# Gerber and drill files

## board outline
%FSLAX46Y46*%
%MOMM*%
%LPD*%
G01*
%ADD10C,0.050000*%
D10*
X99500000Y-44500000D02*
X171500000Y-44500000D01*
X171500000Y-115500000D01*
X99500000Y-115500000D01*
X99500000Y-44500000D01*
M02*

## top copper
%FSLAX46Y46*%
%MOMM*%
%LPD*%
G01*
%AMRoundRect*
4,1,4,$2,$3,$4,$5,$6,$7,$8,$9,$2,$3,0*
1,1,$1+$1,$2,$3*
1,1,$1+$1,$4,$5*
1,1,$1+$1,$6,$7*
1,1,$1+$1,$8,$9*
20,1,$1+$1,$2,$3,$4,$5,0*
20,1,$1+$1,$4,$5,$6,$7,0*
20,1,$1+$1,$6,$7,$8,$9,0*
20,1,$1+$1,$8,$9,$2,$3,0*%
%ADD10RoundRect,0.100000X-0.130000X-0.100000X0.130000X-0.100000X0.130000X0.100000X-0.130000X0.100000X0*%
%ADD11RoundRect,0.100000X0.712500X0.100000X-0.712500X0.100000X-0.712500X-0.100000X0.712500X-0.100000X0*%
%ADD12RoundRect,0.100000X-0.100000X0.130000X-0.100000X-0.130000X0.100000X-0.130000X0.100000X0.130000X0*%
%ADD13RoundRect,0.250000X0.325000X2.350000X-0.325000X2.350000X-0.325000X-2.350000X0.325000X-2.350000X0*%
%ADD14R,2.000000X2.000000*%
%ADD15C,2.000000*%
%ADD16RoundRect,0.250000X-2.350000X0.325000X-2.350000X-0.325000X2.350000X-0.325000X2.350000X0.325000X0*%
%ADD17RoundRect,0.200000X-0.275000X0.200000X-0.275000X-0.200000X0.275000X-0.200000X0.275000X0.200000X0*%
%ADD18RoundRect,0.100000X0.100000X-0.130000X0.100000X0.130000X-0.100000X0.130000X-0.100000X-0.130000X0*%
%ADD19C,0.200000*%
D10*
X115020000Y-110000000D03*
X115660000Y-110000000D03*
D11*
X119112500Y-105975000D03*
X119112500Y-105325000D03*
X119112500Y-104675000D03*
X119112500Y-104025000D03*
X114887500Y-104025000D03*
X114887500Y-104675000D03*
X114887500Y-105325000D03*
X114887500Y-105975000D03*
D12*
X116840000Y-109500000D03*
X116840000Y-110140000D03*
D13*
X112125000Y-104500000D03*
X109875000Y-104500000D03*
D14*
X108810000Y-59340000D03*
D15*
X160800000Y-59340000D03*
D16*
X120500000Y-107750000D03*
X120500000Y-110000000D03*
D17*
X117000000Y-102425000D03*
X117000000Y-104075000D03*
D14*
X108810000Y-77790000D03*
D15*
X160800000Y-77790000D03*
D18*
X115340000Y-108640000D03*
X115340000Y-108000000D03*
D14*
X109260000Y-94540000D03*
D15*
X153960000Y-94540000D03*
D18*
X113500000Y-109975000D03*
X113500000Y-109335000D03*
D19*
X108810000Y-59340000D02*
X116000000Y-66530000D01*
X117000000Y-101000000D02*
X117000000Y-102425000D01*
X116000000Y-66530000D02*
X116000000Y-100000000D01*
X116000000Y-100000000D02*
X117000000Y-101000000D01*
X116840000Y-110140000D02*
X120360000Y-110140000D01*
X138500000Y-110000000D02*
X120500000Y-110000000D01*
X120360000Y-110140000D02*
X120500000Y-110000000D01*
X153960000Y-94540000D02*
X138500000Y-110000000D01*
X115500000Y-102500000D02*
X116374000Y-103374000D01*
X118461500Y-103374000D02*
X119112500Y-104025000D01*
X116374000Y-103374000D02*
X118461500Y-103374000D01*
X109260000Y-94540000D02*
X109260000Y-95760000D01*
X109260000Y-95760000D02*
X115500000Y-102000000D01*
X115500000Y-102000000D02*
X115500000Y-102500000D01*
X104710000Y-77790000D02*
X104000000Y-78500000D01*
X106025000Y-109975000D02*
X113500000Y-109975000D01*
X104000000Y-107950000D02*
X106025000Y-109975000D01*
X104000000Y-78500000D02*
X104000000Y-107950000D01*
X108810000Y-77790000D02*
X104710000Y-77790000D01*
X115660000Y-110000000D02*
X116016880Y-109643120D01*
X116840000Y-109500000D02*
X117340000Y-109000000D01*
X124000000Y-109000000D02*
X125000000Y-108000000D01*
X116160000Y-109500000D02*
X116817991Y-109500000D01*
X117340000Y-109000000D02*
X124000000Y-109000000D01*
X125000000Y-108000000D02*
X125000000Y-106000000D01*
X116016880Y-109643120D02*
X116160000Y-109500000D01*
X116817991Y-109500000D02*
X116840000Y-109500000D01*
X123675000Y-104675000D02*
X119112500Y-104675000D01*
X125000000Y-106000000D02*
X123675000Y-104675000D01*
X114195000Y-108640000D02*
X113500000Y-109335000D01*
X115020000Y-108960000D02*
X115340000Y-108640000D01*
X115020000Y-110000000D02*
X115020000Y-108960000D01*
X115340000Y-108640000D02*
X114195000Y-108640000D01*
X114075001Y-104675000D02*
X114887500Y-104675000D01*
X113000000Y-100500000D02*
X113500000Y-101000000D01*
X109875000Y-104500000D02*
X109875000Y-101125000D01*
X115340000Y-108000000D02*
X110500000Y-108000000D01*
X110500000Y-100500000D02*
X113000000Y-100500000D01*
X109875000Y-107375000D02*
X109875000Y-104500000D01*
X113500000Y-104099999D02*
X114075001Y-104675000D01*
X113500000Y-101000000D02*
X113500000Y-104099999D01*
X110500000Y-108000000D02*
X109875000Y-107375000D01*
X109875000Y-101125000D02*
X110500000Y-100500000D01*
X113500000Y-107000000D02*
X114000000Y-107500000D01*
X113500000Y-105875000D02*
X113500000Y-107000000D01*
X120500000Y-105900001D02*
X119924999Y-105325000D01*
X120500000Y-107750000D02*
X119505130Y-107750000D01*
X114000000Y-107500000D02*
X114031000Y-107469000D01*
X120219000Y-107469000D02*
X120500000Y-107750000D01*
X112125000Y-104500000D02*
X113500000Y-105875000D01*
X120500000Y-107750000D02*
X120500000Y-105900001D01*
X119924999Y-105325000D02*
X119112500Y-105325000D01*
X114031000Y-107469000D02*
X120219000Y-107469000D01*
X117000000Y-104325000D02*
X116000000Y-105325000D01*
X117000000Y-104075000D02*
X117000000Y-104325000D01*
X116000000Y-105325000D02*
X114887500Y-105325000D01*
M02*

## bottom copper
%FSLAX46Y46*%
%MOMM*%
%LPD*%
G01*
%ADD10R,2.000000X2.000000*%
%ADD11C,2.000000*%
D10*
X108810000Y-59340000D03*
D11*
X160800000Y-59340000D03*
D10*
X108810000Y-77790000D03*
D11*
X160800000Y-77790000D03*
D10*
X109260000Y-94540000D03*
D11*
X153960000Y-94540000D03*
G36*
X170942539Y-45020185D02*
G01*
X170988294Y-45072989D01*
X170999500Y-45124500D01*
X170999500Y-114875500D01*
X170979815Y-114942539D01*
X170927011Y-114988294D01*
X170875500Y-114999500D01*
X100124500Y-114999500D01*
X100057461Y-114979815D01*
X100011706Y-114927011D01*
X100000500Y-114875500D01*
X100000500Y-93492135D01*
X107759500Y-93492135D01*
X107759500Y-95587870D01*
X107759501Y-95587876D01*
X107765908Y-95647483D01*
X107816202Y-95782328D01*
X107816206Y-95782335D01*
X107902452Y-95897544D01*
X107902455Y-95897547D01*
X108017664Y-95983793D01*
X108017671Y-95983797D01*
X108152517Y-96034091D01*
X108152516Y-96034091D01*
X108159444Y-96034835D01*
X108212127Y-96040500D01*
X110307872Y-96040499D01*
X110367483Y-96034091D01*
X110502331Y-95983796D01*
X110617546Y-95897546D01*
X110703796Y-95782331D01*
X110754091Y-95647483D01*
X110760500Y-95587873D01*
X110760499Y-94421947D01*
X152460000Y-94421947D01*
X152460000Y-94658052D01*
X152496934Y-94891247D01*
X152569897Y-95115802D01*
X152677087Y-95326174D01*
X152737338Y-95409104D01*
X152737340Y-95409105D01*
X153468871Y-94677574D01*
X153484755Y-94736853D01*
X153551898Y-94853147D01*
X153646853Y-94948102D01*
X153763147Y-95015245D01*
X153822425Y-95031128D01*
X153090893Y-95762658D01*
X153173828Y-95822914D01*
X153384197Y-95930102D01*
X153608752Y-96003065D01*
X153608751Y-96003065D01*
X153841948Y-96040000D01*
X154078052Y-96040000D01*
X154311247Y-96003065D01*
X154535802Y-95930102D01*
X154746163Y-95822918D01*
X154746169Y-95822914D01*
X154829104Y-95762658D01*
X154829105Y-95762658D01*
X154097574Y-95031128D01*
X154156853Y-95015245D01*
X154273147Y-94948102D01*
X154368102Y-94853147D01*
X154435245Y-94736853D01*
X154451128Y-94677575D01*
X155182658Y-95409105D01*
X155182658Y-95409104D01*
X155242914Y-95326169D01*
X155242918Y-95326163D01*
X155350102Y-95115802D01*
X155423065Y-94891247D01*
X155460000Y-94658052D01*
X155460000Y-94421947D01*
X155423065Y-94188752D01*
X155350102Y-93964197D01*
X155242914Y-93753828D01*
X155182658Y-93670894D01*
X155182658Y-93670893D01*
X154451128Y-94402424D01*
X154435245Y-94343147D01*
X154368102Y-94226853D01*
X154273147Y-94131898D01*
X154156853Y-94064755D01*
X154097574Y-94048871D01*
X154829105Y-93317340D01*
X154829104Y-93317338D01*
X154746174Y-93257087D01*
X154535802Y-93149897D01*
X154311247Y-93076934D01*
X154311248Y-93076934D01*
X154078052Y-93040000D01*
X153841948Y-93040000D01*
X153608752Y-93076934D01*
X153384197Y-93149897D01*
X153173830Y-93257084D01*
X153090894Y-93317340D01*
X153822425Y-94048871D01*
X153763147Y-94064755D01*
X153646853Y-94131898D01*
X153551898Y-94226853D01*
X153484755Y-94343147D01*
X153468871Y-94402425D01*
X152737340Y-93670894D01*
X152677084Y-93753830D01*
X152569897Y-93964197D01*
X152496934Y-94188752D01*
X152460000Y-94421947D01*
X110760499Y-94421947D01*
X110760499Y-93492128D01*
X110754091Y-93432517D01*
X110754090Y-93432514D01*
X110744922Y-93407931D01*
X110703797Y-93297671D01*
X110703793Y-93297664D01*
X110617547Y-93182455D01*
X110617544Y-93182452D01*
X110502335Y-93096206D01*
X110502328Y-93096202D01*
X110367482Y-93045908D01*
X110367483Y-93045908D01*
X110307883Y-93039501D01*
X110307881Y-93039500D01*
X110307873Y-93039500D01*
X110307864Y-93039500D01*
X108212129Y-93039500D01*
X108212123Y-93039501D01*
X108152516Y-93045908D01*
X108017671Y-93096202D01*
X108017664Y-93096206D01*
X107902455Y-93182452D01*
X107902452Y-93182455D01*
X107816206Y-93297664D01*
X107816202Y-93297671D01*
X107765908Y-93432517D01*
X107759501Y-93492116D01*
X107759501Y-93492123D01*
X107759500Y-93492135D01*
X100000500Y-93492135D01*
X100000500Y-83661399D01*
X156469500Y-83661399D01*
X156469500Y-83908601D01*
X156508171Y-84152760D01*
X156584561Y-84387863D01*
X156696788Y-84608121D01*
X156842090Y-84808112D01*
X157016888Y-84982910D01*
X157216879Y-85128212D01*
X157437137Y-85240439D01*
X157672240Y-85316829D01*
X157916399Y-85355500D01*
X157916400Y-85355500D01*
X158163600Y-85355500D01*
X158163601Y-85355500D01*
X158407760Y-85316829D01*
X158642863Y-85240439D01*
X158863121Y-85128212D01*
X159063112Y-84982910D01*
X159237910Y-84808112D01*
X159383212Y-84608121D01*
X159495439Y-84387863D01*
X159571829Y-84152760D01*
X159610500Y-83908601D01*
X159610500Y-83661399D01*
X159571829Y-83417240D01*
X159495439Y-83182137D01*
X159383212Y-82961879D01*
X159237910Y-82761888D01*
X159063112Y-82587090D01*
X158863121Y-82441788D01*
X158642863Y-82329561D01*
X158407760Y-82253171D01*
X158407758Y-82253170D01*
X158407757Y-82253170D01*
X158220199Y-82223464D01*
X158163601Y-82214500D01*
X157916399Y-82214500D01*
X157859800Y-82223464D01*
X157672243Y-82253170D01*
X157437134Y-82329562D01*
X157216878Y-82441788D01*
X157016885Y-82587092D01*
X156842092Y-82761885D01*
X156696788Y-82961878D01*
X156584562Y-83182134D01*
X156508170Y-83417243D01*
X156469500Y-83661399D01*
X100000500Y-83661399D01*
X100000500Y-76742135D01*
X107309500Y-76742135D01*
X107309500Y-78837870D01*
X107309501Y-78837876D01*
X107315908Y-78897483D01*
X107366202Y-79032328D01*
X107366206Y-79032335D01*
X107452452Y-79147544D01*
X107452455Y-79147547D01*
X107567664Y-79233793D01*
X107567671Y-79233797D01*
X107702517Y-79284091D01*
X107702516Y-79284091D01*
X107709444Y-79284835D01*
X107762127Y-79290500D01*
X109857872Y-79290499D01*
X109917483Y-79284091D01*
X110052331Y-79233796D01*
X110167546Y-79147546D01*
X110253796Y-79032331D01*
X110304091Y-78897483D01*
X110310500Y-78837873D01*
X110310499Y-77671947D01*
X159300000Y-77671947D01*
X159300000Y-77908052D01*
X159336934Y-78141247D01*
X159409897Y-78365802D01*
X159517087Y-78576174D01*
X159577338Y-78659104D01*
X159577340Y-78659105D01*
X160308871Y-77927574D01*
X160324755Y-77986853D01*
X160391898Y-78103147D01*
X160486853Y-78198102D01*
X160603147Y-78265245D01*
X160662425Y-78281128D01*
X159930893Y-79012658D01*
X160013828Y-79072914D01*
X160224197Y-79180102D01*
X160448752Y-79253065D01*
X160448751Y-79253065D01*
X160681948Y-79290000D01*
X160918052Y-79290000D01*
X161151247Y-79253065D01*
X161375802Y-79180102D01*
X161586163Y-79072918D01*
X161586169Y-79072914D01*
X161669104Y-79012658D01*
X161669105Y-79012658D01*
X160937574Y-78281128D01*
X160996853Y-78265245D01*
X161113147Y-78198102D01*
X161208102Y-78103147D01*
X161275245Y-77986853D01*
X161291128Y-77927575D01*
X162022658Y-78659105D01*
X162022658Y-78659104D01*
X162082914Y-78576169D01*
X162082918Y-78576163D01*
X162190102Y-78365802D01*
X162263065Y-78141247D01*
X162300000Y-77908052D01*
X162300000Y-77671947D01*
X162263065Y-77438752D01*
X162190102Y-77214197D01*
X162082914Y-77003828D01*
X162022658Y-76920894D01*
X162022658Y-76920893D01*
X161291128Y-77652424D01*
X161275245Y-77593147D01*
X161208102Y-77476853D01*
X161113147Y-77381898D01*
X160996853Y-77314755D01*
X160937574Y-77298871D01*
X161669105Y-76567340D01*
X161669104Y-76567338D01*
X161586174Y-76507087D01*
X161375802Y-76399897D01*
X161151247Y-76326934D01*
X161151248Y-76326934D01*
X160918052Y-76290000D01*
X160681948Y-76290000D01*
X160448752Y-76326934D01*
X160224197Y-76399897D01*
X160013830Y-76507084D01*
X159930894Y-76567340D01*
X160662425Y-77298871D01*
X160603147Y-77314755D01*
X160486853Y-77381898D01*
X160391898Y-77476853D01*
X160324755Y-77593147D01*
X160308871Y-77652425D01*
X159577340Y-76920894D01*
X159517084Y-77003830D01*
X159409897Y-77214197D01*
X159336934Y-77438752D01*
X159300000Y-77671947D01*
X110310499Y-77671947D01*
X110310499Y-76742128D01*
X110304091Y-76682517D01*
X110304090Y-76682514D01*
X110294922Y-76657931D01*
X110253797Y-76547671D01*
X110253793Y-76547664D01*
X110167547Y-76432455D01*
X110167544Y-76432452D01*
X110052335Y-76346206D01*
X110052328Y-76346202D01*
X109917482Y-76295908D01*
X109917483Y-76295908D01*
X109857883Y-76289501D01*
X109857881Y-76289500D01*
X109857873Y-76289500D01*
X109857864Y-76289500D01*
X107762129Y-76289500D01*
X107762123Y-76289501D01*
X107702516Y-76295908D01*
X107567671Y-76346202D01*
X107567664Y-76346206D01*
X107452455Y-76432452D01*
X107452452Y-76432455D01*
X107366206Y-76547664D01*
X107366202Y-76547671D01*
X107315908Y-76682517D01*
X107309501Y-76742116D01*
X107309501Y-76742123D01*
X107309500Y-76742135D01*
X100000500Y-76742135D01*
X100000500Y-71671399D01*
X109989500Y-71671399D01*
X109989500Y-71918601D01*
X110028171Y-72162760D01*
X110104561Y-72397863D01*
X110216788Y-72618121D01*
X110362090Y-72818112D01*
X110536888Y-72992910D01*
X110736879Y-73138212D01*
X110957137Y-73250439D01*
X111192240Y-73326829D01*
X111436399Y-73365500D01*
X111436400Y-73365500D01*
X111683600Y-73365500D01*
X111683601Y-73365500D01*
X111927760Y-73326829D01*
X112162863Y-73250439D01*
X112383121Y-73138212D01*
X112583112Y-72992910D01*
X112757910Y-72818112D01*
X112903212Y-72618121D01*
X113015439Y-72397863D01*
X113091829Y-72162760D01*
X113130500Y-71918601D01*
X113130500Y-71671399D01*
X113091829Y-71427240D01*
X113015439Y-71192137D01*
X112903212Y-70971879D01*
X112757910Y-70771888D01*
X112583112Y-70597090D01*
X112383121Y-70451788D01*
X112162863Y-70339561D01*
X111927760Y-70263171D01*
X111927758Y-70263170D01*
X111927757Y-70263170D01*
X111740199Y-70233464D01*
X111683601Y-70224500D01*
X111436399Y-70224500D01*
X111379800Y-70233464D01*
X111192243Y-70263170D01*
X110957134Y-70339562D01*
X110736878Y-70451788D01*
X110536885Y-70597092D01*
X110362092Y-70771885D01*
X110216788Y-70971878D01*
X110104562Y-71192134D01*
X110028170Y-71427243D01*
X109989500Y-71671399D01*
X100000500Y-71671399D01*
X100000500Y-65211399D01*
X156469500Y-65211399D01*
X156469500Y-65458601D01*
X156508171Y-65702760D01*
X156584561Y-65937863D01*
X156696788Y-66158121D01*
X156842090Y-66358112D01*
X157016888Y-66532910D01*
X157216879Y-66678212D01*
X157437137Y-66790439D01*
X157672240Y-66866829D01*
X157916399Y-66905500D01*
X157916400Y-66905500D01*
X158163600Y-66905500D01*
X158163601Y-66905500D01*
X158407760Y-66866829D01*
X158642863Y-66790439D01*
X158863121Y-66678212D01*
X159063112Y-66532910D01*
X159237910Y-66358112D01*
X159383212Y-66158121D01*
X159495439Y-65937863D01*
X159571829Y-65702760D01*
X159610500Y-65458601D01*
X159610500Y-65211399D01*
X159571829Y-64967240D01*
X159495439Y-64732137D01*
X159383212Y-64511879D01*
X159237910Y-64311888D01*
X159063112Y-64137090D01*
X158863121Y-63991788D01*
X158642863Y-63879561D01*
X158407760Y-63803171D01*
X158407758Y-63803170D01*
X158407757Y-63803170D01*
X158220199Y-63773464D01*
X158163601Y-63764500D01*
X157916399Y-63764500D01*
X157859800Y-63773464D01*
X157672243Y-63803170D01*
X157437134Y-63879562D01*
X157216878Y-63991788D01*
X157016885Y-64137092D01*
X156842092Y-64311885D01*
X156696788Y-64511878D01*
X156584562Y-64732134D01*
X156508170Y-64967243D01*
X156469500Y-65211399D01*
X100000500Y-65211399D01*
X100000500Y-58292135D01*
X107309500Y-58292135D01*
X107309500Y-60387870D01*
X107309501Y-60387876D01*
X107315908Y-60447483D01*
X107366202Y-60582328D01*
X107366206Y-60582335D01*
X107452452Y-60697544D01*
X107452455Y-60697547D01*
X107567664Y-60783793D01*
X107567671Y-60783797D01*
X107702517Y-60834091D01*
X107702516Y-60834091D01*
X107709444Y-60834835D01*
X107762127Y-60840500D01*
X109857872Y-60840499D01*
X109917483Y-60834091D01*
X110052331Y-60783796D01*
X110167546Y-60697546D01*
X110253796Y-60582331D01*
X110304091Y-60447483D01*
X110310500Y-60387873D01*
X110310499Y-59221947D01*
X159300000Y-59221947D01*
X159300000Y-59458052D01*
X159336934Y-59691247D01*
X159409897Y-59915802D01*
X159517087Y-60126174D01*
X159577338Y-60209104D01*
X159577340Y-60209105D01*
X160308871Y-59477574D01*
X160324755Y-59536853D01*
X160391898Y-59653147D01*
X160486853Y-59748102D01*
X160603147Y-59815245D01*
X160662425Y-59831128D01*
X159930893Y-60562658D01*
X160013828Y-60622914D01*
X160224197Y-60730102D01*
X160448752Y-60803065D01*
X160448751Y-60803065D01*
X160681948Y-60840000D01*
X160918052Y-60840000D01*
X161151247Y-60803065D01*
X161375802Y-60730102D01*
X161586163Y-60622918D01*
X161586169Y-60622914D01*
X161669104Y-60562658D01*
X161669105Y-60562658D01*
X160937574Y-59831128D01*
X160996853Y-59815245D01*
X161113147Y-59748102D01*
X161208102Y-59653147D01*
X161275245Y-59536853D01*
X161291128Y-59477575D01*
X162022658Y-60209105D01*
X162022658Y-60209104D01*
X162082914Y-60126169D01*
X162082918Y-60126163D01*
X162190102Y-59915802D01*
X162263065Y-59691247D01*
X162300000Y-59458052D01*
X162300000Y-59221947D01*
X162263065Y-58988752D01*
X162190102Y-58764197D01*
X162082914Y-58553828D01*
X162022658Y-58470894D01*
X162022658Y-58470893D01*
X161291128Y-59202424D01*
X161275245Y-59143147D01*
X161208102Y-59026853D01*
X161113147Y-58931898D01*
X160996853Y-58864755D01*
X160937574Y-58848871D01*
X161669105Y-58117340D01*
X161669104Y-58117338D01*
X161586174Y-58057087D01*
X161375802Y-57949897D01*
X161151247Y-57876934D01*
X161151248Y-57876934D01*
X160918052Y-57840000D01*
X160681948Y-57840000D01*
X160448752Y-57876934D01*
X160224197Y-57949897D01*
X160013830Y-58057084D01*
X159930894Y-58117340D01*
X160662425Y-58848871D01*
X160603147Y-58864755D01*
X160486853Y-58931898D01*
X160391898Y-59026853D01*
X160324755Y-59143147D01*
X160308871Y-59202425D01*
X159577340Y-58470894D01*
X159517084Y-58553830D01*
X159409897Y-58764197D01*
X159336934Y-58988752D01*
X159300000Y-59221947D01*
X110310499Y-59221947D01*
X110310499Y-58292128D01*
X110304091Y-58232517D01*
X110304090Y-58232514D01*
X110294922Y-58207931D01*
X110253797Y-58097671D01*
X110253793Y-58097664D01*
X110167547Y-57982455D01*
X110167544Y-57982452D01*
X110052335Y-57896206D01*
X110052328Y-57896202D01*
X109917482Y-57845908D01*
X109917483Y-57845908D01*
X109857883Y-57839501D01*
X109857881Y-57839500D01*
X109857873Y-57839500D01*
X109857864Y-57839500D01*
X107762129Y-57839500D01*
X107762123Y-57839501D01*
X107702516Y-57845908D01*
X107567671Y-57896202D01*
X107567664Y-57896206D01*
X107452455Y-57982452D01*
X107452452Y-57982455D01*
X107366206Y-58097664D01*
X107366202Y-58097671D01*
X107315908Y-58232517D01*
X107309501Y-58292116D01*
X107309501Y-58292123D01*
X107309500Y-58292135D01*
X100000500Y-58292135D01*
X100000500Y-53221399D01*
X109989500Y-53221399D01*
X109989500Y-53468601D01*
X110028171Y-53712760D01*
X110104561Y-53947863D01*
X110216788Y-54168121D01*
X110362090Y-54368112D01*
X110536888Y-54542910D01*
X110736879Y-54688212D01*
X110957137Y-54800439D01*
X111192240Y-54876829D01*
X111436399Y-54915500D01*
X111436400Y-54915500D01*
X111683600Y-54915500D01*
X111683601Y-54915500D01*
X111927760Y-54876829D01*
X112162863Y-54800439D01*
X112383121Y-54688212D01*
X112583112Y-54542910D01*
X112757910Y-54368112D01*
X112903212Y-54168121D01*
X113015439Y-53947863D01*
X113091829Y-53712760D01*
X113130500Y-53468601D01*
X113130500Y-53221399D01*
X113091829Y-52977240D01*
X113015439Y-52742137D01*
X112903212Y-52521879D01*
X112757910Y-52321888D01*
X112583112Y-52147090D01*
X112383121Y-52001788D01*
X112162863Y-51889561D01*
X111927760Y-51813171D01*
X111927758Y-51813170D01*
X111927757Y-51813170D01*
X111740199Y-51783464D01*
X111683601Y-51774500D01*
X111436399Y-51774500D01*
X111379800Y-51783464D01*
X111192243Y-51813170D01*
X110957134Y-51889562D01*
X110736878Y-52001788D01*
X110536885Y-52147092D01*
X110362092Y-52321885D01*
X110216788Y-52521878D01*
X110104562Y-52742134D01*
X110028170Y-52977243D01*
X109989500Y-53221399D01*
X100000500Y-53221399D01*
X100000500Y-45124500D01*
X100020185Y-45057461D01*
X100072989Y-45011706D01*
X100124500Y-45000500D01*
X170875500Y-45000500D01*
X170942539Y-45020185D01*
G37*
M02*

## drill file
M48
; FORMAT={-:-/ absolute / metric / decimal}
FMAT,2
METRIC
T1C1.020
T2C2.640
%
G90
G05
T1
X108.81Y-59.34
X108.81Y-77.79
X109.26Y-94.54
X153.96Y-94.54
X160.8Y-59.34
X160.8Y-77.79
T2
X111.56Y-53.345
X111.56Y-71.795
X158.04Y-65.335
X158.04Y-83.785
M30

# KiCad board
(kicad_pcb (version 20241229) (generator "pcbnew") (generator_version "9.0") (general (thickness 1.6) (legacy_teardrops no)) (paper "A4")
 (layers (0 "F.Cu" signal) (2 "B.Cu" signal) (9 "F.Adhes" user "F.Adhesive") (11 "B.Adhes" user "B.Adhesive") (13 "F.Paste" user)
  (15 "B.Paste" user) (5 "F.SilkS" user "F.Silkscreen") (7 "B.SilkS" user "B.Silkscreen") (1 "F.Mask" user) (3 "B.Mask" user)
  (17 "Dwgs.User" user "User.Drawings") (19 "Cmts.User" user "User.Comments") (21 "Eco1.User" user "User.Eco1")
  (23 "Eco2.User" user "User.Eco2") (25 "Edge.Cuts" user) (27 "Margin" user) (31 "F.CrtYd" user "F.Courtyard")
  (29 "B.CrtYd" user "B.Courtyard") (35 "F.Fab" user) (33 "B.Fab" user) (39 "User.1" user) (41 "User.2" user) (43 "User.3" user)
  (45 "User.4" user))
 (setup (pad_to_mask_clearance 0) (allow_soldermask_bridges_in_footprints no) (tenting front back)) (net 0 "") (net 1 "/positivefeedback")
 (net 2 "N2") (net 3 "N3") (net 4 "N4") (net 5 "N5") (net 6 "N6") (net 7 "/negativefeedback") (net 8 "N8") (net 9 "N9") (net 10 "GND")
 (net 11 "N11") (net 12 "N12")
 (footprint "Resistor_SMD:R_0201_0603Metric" (layer "F.Cu") (at 115.34 110)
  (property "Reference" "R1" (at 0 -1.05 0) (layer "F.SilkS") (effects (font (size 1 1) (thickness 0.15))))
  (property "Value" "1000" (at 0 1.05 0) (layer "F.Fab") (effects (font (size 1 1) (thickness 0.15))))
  (pad "" smd roundrect (at -0.345 0) (size 0.318 0.36) (layers "F.Paste") (roundrect_rratio 0.25))
  (pad "" smd roundrect (at 0.345 0) (size 0.318 0.36) (layers "F.Paste") (roundrect_rratio 0.25))
  (pad "1" smd roundrect (at -0.32 0) (size 0.46 0.4) (layers "F.Cu" "F.Mask") (roundrect_rratio 0.25) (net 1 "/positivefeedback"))
  (pad "2" smd roundrect (at 0.32 0) (size 0.46 0.4) (layers "F.Cu" "F.Mask") (roundrect_rratio 0.25) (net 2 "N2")))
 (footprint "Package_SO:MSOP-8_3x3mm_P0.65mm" (layer "F.Cu") (at 117 105 180)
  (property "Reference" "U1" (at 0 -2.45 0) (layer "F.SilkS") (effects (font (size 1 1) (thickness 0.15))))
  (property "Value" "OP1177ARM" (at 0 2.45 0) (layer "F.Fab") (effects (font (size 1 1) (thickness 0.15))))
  (pad "1" smd roundrect (at -2.1125 -0.975 180) (size 1.625 0.4) (layers "F.Cu" "F.Mask" "F.Paste") (roundrect_rratio 0.25) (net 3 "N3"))
  (pad "2" smd roundrect (at -2.1125 -0.325 180) (size 1.625 0.4) (layers "F.Cu" "F.Mask" "F.Paste") (roundrect_rratio 0.25) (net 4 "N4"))
  (pad "3" smd roundrect (at -2.1125 0.325 180) (size 1.625 0.4) (layers "F.Cu" "F.Mask" "F.Paste") (roundrect_rratio 0.25) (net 2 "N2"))
  (pad "4" smd roundrect (at -2.1125 0.975 180) (size 1.625 0.4) (layers "F.Cu" "F.Mask" "F.Paste") (roundrect_rratio 0.25) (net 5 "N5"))
  (pad "5" smd roundrect (at 2.1125 0.975 180) (size 1.625 0.4) (layers "F.Cu" "F.Mask" "F.Paste") (roundrect_rratio 0.25) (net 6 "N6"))
  (pad "6" smd roundrect (at 2.1125 0.325 180) (size 1.625 0.4) (layers "F.Cu" "F.Mask" "F.Paste") (roundrect_rratio 0.25)
   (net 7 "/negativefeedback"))
  (pad "7" smd roundrect (at 2.1125 -0.325 180) (size 1.625 0.4) (layers "F.Cu" "F.Mask" "F.Paste") (roundrect_rratio 0.25) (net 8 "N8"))
  (pad "8" smd roundrect (at 2.1125 -0.975 180) (size 1.625 0.4) (layers "F.Cu" "F.Mask" "F.Paste") (roundrect_rratio 0.25) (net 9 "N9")))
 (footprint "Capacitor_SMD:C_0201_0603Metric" (layer "F.Cu") (at 116.84 109.82 -90)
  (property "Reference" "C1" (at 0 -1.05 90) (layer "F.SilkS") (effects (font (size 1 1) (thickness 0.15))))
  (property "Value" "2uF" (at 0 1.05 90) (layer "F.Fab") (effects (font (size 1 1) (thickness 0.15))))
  (pad "" smd roundrect (at -0.345 0 270) (size 0.318 0.36) (layers "F.Paste") (roundrect_rratio 0.25))
  (pad "" smd roundrect (at 0.345 0 270) (size 0.318 0.36) (layers "F.Paste") (roundrect_rratio 0.25))
  (pad "1" smd roundrect (at -0.32 0 270) (size 0.46 0.4) (layers "F.Cu" "F.Mask") (roundrect_rratio 0.25) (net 2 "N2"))
  (pad "2" smd roundrect (at 0.32 0 270) (size 0.46 0.4) (layers "F.Cu" "F.Mask") (roundrect_rratio 0.25) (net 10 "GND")))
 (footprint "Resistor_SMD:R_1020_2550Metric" (layer "F.Cu") (at 111 104.5 180)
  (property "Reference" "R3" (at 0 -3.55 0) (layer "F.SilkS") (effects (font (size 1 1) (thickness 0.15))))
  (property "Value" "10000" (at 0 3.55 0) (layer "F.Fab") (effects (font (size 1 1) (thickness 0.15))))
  (pad "1" smd roundrect (at -1.125 0 180) (size 1.15 5.2) (layers "F.Cu" "F.Mask" "F.Paste") (roundrect_rratio 0.217391) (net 4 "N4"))
  (pad "2" smd roundrect (at 1.125 0 180) (size 1.15 5.2) (layers "F.Cu" "F.Mask" "F.Paste") (roundrect_rratio 0.217391)
   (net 7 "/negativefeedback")))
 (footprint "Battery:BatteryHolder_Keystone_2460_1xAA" (layer "F.Cu") (at 108.81 59.34)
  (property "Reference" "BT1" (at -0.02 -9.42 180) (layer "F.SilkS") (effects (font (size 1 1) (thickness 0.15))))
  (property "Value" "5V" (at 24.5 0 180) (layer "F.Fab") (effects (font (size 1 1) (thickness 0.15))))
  (pad "" np_thru_hole circle (at 2.75 -5.995 90) (size 2.64 2.64) (drill 2.64) (layers "*.Cu" "*.Mask"))
  (pad "" np_thru_hole circle (at 49.23 5.995) (size 2.64 2.64) (drill 2.64) (layers "*.Cu" "*.Mask"))
  (pad "1" thru_hole rect (at 0 0 180) (size 2 2) (drill 1.02) (layers "*.Cu" "*.Mask") (remove_unused_layers no) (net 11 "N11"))
  (pad "2" thru_hole circle (at 51.99 0 180) (size 2 2) (drill 1.02) (layers "*.Cu" "*.Mask") (remove_unused_layers no) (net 10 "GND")))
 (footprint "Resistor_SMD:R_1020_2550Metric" (layer "F.Cu") (at 120.5 108.875 -90)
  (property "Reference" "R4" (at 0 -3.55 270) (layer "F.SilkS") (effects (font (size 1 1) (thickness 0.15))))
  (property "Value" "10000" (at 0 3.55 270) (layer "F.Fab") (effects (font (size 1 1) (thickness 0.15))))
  (pad "1" smd roundrect (at -1.125 0 270) (size 1.15 5.2) (layers "F.Cu" "F.Mask" "F.Paste") (roundrect_rratio 0.217391) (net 4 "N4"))
  (pad "2" smd roundrect (at 1.125 0 270) (size 1.15 5.2) (layers "F.Cu" "F.Mask" "F.Paste") (roundrect_rratio 0.217391) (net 10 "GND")))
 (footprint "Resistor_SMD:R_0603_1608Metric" (layer "F.Cu") (at 117 103.25 -90)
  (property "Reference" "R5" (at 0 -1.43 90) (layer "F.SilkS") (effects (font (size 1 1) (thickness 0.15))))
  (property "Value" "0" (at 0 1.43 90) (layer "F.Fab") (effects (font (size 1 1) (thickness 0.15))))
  (pad "1" smd roundrect (at -0.825 0 270) (size 0.8 0.95) (layers "F.Cu" "F.Mask" "F.Paste") (roundrect_rratio 0.25) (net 11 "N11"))
  (pad "2" smd roundrect (at 0.825 0 270) (size 0.8 0.95) (layers "F.Cu" "F.Mask" "F.Paste") (roundrect_rratio 0.25) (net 8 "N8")))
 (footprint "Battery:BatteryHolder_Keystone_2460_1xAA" (layer "F.Cu") (at 108.81 77.79)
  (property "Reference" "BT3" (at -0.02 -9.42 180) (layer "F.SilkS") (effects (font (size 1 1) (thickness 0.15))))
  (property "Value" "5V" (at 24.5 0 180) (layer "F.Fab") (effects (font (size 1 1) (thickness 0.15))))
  (pad "" np_thru_hole circle (at 2.75 -5.995 90) (size 2.64 2.64) (drill 2.64) (layers "*.Cu" "*.Mask"))
  (pad "" np_thru_hole circle (at 49.23 5.995) (size 2.64 2.64) (drill 2.64) (layers "*.Cu" "*.Mask"))
  (pad "1" thru_hole rect (at 0 0 180) (size 2 2) (drill 1.02) (layers "*.Cu" "*.Mask") (remove_unused_layers no) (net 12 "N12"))
  (pad "2" thru_hole circle (at 51.99 0 180) (size 2 2) (drill 1.02) (layers "*.Cu" "*.Mask") (remove_unused_layers no) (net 10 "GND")))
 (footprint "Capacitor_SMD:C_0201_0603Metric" (layer "F.Cu") (at 115.34 108.32 90)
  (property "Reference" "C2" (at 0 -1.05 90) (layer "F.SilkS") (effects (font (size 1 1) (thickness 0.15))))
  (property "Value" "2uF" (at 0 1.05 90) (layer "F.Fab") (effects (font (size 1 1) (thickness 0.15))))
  (pad "" smd roundrect (at -0.345 0 90) (size 0.318 0.36) (layers "F.Paste") (roundrect_rratio 0.25))
  (pad "" smd roundrect (at 0.345 0 90) (size 0.318 0.36) (layers "F.Paste") (roundrect_rratio 0.25))
  (pad "1" smd roundrect (at -0.32 0 90) (size 0.46 0.4) (layers "F.Cu" "F.Mask") (roundrect_rratio 0.25) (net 1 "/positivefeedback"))
  (pad "2" smd roundrect (at 0.32 0 90) (size 0.46 0.4) (layers "F.Cu" "F.Mask") (roundrect_rratio 0.25) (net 7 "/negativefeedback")))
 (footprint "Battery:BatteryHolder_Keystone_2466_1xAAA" (layer "F.Cu") (at 109.26 94.54)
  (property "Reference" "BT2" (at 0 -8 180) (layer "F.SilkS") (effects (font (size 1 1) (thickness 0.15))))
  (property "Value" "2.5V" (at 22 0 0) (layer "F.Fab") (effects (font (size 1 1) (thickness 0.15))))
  (pad "1" thru_hole rect (at 0 0) (size 2 2) (drill 1.02) (layers "*.Cu" "*.Mask") (remove_unused_layers no) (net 5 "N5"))
  (pad "2" thru_hole circle (at 44.7 0) (size 2 2) (drill 1.02) (layers "*.Cu" "*.Mask") (remove_unused_layers no) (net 10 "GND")))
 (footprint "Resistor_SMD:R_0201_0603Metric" (layer "F.Cu") (at 113.5 109.655 90)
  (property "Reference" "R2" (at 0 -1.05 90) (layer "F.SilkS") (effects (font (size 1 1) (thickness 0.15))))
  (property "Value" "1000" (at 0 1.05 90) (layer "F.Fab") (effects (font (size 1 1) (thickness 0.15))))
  (pad "" smd roundrect (at -0.345 0 90) (size 0.318 0.36) (layers "F.Paste") (roundrect_rratio 0.25))
  (pad "" smd roundrect (at 0.345 0 90) (size 0.318 0.36) (layers "F.Paste") (roundrect_rratio 0.25))
  (pad "1" smd roundrect (at -0.32 0 90) (size 0.46 0.4) (layers "F.Cu" "F.Mask") (roundrect_rratio 0.25) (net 12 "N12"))
  (pad "2" smd roundrect (at 0.32 0 90) (size 0.46 0.4) (layers "F.Cu" "F.Mask") (roundrect_rratio 0.25) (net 1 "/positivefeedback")))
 (gr_rect (start 99.5 44.5) (end 171.5 115.5) (stroke (width 0.05) (type default)) (fill no) (layer "Edge.Cuts"))
 (segment (start 108.81 59.34) (end 116 66.53) (width 0.2) (layer "F.Cu") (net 11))
 (segment (start 117 101) (end 117 102.425) (width 0.2) (layer "F.Cu") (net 11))
 (segment (start 116 66.53) (end 116 100) (width 0.2) (layer "F.Cu") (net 11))
 (segment (start 116 100) (end 117 101) (width 0.2) (layer "F.Cu") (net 11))
 (segment (start 116.84 110.14) (end 120.36 110.14) (width 0.2) (layer "F.Cu") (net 10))
 (segment (start 138.5 110) (end 120.5 110) (width 0.2) (layer "F.Cu") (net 10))
 (segment (start 120.36 110.14) (end 120.5 110) (width 0.2) (layer "F.Cu") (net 10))
 (segment (start 153.96 94.54) (end 138.5 110) (width 0.2) (layer "F.Cu") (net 10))
 (segment (start 115.5 102.5) (end 116.374 103.374) (width 0.2) (layer "F.Cu") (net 5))
 (segment (start 118.4615 103.374) (end 119.1125 104.025) (width 0.2) (layer "F.Cu") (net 5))
 (segment (start 116.374 103.374) (end 118.4615 103.374) (width 0.2) (layer "F.Cu") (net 5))
 (segment (start 109.26 94.54) (end 109.26 95.76) (width 0.2) (layer "F.Cu") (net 5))
 (segment (start 109.26 95.76) (end 115.5 102) (width 0.2) (layer "F.Cu") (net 5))
 (segment (start 115.5 102) (end 115.5 102.5) (width 0.2) (layer "F.Cu") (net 5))
 (segment (start 104.71 77.79) (end 104 78.5) (width 0.2) (layer "F.Cu") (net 12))
 (segment (start 106.025 109.975) (end 113.5 109.975) (width 0.2) (layer "F.Cu") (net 12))
 (segment (start 104 107.95) (end 106.025 109.975) (width 0.2) (layer "F.Cu") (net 12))
 (segment (start 104 78.5) (end 104 107.95) (width 0.2) (layer "F.Cu") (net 12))
 (segment (start 108.81 77.79) (end 104.71 77.79) (width 0.2) (layer "F.Cu") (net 12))
 (segment (start 115.66 110) (end 116.01688 109.64312) (width 0.2) (layer "F.Cu") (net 2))
 (segment (start 116.84 109.5) (end 117.34 109) (width 0.2) (layer "F.Cu") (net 2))
 (segment (start 124 109) (end 125 108) (width 0.2) (layer "F.Cu") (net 2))
 (segment (start 116.16 109.5) (end 116.817991 109.5) (width 0.2) (layer "F.Cu") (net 2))
 (segment (start 117.34 109) (end 124 109) (width 0.2) (layer "F.Cu") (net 2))
 (segment (start 125 108) (end 125 106) (width 0.2) (layer "F.Cu") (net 2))
 (segment (start 116.01688 109.64312) (end 116.16 109.5) (width 0.2) (layer "F.Cu") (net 2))
 (segment (start 116.817991 109.5) (end 116.84 109.5) (width 0.2) (layer "F.Cu") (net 2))
 (segment (start 123.675 104.675) (end 119.1125 104.675) (width 0.2) (layer "F.Cu") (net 2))
 (segment (start 125 106) (end 123.675 104.675) (width 0.2) (layer "F.Cu") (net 2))
 (segment (start 114.195 108.64) (end 113.5 109.335) (width 0.2) (layer "F.Cu") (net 1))
 (segment (start 115.02 108.96) (end 115.34 108.64) (width 0.2) (layer "F.Cu") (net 1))
 (segment (start 115.02 110) (end 115.02 108.96) (width 0.2) (layer "F.Cu") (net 1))
 (segment (start 115.34 108.64) (end 114.195 108.64) (width 0.2) (layer "F.Cu") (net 1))
 (segment (start 114.075001 104.675) (end 114.8875 104.675) (width 0.2) (layer "F.Cu") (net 7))
 (segment (start 113 100.5) (end 113.5 101) (width 0.2) (layer "F.Cu") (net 7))
 (segment (start 109.875 104.5) (end 109.875 101.125) (width 0.2) (layer "F.Cu") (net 7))
 (segment (start 115.34 108) (end 110.5 108) (width 0.2) (layer "F.Cu") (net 7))
 (segment (start 110.5 100.5) (end 113 100.5) (width 0.2) (layer "F.Cu") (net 7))
 (segment (start 109.875 107.375) (end 109.875 104.5) (width 0.2) (layer "F.Cu") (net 7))
 (segment (start 113.5 104.099999) (end 114.075001 104.675) (width 0.2) (layer "F.Cu") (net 7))
 (segment (start 113.5 101) (end 113.5 104.099999) (width 0.2) (layer "F.Cu") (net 7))
 (segment (start 110.5 108) (end 109.875 107.375) (width 0.2) (layer "F.Cu") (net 7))
 (segment (start 109.875 101.125) (end 110.5 100.5) (width 0.2) (layer "F.Cu") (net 7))
 (segment (start 113.5 107) (end 114 107.5) (width 0.2) (layer "F.Cu") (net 4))
 (segment (start 113.5 105.875) (end 113.5 107) (width 0.2) (layer "F.Cu") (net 4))
 (segment (start 120.5 105.900001) (end 119.924999 105.325) (width 0.2) (layer "F.Cu") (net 4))
 (segment (start 120.5 107.75) (end 119.50513 107.75) (width 0.2) (layer "F.Cu") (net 4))
 (segment (start 114 107.5) (end 114.031 107.469) (width 0.2) (layer "F.Cu") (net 4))
 (segment (start 120.219 107.469) (end 120.5 107.75) (width 0.2) (layer "F.Cu") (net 4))
 (segment (start 112.125 104.5) (end 113.5 105.875) (width 0.2) (layer "F.Cu") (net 4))
 (segment (start 120.5 107.75) (end 120.5 105.900001) (width 0.2) (layer "F.Cu") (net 4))
 (segment (start 119.924999 105.325) (end 119.1125 105.325) (width 0.2) (layer "F.Cu") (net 4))
 (segment (start 114.031 107.469) (end 120.219 107.469) (width 0.2) (layer "F.Cu") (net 4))
 (segment (start 117 104.325) (end 116 105.325) (width 0.2) (layer "F.Cu") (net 8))
 (segment (start 117 104.075) (end 117 104.325) (width 0.2) (layer "F.Cu") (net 8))
 (segment (start 116 105.325) (end 114.8875 105.325) (width 0.2) (layer "F.Cu") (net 8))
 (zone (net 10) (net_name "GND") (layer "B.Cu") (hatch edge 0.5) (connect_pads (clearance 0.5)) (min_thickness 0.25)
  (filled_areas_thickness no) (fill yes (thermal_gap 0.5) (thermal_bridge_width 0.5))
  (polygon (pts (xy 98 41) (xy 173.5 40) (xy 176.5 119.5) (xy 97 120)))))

